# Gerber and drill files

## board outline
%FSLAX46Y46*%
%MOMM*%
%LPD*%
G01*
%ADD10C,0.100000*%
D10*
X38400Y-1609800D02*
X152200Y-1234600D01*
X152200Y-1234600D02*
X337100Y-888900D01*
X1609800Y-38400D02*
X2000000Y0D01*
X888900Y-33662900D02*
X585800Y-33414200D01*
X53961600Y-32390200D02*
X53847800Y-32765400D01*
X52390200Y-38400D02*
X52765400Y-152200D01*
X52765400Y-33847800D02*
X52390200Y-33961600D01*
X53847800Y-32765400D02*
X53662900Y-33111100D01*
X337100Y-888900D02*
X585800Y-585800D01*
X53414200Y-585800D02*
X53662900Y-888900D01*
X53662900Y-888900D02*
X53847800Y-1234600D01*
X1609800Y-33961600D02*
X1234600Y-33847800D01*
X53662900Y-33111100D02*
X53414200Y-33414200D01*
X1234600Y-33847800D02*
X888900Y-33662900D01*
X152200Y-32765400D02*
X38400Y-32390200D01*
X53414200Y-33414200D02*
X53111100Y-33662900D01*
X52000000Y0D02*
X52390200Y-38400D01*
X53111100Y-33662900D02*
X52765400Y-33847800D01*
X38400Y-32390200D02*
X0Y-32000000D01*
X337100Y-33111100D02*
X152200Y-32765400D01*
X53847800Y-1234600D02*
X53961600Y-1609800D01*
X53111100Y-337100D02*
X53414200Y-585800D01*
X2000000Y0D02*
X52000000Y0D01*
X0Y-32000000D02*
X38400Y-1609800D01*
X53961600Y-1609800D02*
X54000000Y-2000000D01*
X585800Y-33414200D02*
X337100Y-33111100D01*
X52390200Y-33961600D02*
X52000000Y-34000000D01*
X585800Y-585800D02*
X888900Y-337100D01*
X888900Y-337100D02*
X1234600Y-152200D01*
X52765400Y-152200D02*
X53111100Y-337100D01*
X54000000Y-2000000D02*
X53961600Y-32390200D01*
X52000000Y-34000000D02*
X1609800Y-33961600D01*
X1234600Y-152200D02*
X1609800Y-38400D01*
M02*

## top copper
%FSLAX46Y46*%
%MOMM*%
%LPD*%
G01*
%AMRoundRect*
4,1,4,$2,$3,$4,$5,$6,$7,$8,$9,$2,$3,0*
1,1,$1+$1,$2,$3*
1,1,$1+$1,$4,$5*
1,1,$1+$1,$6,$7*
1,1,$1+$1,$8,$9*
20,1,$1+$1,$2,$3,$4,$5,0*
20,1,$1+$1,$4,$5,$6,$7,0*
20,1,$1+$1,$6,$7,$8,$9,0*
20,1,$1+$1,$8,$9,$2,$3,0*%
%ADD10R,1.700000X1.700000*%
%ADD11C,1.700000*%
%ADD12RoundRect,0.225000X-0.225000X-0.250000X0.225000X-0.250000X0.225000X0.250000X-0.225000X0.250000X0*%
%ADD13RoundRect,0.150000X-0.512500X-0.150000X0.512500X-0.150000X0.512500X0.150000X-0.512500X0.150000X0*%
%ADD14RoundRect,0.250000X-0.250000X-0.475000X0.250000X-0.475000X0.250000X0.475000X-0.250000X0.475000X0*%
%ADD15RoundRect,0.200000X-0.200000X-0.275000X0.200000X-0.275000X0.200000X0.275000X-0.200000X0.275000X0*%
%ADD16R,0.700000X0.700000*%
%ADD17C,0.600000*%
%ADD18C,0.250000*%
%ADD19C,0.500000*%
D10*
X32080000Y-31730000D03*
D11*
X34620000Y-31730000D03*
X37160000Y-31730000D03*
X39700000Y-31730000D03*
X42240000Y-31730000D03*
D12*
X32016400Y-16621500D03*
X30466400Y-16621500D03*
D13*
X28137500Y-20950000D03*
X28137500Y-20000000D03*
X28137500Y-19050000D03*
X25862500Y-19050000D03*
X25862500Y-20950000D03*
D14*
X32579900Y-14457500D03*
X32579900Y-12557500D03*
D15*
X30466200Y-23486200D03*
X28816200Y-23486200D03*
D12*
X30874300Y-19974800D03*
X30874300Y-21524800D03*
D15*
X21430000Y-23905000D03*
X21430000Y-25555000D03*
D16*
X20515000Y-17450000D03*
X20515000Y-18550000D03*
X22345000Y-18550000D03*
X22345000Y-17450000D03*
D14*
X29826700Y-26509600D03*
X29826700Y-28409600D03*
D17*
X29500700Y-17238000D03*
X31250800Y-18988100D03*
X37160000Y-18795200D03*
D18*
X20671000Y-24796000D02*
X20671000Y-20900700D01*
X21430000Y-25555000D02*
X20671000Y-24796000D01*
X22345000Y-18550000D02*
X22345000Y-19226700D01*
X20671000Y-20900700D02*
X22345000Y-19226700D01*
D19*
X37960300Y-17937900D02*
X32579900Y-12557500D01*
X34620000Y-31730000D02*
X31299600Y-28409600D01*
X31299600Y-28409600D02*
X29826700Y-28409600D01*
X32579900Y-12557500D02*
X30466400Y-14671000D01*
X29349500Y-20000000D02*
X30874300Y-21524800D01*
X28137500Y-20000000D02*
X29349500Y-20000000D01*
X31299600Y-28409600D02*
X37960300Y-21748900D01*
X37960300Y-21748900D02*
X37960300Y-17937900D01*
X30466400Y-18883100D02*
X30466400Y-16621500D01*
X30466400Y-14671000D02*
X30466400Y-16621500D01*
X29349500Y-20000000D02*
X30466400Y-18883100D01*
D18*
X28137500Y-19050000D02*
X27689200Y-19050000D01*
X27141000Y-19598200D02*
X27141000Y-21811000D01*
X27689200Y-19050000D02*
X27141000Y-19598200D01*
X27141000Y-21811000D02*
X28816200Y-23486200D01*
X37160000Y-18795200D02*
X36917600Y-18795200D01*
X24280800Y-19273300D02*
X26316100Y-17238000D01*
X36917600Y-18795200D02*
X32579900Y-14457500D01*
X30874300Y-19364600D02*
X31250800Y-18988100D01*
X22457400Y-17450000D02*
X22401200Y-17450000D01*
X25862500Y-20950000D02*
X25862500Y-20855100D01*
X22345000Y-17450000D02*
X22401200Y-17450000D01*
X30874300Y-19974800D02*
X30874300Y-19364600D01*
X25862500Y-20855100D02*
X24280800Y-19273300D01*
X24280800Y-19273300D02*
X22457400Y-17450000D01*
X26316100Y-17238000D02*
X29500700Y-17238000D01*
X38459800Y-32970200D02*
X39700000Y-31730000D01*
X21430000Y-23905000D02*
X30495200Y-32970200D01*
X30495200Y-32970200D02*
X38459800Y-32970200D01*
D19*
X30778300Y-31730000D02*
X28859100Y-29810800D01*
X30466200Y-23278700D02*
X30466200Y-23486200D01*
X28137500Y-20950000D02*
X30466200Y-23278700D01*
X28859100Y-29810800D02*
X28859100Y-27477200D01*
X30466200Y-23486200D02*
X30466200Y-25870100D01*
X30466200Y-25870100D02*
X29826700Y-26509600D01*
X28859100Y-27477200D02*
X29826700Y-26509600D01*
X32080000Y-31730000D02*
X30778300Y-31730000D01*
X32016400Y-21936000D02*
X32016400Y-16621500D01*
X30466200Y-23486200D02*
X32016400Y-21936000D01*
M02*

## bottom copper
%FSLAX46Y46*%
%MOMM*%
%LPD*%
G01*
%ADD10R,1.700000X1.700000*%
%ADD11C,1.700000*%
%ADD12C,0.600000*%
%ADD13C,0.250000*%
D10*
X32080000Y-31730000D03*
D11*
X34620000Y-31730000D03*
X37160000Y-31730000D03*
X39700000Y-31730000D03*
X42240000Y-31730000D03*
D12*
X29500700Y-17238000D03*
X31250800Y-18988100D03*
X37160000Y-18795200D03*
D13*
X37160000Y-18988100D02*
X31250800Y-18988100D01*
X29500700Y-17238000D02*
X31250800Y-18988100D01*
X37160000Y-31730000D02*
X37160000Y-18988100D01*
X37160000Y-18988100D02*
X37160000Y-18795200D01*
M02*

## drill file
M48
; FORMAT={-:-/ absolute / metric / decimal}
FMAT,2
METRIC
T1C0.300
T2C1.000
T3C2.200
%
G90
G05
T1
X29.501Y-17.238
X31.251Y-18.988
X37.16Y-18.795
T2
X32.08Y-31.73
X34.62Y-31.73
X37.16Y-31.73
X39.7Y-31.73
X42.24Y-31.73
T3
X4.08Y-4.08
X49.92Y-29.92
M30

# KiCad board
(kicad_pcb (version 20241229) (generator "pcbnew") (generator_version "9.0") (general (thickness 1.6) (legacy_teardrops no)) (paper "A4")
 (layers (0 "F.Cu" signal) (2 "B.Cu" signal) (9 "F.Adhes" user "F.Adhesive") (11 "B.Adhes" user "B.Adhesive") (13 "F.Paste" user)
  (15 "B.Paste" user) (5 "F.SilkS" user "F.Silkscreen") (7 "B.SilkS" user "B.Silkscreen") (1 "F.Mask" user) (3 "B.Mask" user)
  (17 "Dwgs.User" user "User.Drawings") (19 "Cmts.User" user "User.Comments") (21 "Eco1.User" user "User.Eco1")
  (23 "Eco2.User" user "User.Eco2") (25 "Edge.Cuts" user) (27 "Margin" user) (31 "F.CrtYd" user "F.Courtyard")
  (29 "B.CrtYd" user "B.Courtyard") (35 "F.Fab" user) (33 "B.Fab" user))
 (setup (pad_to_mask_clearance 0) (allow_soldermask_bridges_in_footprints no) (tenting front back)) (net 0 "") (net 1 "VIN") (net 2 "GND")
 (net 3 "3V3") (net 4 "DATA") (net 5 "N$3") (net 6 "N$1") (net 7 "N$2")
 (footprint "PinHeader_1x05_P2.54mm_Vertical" (layer "F.Cu") (at 32.08 31.73 90)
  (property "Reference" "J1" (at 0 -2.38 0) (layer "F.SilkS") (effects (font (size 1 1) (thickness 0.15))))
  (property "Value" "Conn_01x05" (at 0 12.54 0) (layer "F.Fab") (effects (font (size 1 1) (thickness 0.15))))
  (pad "1" thru_hole rect (at 0 0) (size 1.7 1.7) (drill 1) (layers "*.Cu" "*.Mask") (remove_unused_layers no) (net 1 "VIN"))
  (pad "2" thru_hole circle (at 0 2.54) (size 1.7 1.7) (drill 1) (layers "*.Cu" "*.Mask") (remove_unused_layers no) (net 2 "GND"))
  (pad "3" thru_hole circle (at 0 5.08) (size 1.7 1.7) (drill 1) (layers "*.Cu" "*.Mask") (remove_unused_layers no) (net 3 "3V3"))
  (pad "4" thru_hole circle (at 0 7.62) (size 1.7 1.7) (drill 1) (layers "*.Cu" "*.Mask") (remove_unused_layers no) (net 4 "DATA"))
  (pad "5" thru_hole circle (at 0 10.16) (size 1.7 1.7) (drill 1) (layers "*.Cu" "*.Mask") (remove_unused_layers no) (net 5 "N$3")))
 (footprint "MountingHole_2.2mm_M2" (layer "F.Cu") (at 4.08 4.08)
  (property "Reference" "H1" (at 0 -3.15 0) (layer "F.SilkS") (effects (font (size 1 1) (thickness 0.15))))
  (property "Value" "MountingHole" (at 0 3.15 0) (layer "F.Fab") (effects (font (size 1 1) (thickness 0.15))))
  (pad "" np_thru_hole circle (at 0 0) (size 2.2 2.2) (drill 2.2) (layers "*.Cu" "*.Mask")))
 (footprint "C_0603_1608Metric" (layer "F.Cu") (at 31.2414 16.6215 180)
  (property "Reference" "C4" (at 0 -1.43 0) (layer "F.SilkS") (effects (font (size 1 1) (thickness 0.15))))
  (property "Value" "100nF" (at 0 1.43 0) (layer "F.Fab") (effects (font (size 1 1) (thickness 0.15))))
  (pad "1" smd roundrect (at -0.775 0) (size 0.9 0.95) (layers "F.Cu" "F.Mask" "F.Paste") (roundrect_rratio 0.25) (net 1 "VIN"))
  (pad "2" smd roundrect (at 0.775 0) (size 0.9 0.95) (layers "F.Cu" "F.Mask" "F.Paste") (roundrect_rratio 0.25) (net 2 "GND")))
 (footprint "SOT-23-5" (layer "F.Cu") (at 27 20 180)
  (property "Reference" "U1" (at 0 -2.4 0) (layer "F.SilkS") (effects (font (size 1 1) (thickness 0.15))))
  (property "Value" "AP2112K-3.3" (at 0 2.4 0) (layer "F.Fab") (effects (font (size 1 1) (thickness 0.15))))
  (pad "1" smd roundrect (at -1.1375 -0.95) (size 1.325 0.6) (layers "F.Cu" "F.Mask" "F.Paste") (roundrect_rratio 0.25) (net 1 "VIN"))
  (pad "2" smd roundrect (at -1.1375 0) (size 1.325 0.6) (layers "F.Cu" "F.Mask" "F.Paste") (roundrect_rratio 0.25) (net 2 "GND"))
  (pad "3" smd roundrect (at -1.1375 0.95) (size 1.325 0.6) (layers "F.Cu" "F.Mask" "F.Paste") (roundrect_rratio 0.25) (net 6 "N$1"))
  (pad "4" smd roundrect (at 1.1375 0.95) (size 1.325 0.6) (layers "F.Cu" "F.Mask" "F.Paste") (roundrect_rratio 0.25))
  (pad "5" smd roundrect (at 1.1375 -0.95) (size 1.325 0.6) (layers "F.Cu" "F.Mask" "F.Paste") (roundrect_rratio 0.25) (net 3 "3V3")))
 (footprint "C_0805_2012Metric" (layer "F.Cu") (at 32.5799 13.5075 90)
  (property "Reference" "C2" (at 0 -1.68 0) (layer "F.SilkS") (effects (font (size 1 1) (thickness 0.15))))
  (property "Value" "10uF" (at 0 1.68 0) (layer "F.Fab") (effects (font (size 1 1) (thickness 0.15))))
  (pad "1" smd roundrect (at -0.95 0) (size 1 1.45) (layers "F.Cu" "F.Mask" "F.Paste") (roundrect_rratio 0.25) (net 3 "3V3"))
  (pad "2" smd roundrect (at 0.95 0) (size 1 1.45) (layers "F.Cu" "F.Mask" "F.Paste") (roundrect_rratio 0.25) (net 2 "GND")))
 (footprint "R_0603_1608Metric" (layer "F.Cu") (at 29.6412 23.4862 180)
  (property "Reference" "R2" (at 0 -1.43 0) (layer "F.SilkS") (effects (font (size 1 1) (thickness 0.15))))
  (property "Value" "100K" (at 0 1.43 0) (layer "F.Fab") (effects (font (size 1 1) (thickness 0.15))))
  (pad "1" smd roundrect (at -0.825 0) (size 0.8 0.95) (layers "F.Cu" "F.Mask" "F.Paste") (roundrect_rratio 0.25) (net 1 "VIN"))
  (pad "2" smd roundrect (at 0.825 0) (size 0.8 0.95) (layers "F.Cu" "F.Mask" "F.Paste") (roundrect_rratio 0.25) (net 6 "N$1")))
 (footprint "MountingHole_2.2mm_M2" (layer "F.Cu") (at 49.92 29.92)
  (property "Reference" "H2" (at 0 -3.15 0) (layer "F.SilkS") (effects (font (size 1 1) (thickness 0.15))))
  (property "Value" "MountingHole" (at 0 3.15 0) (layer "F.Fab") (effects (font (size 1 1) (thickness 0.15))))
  (pad "" np_thru_hole circle (at 0 0) (size 2.2 2.2) (drill 2.2) (layers "*.Cu" "*.Mask")))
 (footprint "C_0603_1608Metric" (layer "F.Cu") (at 30.8743 20.7498 -90)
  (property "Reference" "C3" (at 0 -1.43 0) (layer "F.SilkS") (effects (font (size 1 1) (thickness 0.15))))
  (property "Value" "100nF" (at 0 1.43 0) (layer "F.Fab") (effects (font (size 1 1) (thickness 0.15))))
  (pad "1" smd roundrect (at -0.775 0) (size 0.9 0.95) (layers "F.Cu" "F.Mask" "F.Paste") (roundrect_rratio 0.25) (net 3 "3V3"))
  (pad "2" smd roundrect (at 0.775 0) (size 0.9 0.95) (layers "F.Cu" "F.Mask" "F.Paste") (roundrect_rratio 0.25) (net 2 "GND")))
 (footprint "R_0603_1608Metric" (layer "F.Cu") (at 21.43 24.73 -90)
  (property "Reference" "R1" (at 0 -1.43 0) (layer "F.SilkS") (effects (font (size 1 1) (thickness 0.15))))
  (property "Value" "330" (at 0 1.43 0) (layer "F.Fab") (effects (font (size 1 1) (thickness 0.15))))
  (pad "1" smd roundrect (at -0.825 0) (size 0.8 0.95) (layers "F.Cu" "F.Mask" "F.Paste") (roundrect_rratio 0.25) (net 4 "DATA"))
  (pad "2" smd roundrect (at 0.825 0) (size 0.8 0.95) (layers "F.Cu" "F.Mask" "F.Paste") (roundrect_rratio 0.25) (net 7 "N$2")))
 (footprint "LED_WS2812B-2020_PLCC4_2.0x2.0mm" (layer "F.Cu") (at 21.43 18)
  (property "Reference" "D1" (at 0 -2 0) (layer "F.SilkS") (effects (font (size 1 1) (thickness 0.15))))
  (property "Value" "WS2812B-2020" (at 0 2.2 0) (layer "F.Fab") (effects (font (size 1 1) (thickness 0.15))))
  (pad "1" smd rect (at -0.915 -0.55) (size 0.7 0.7) (layers "F.Cu" "F.Mask" "F.Paste") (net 5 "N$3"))
  (pad "2" smd rect (at -0.915 0.55) (size 0.7 0.7) (layers "F.Cu" "F.Mask" "F.Paste") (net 2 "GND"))
  (pad "3" smd rect (at 0.915 0.55) (size 0.7 0.7) (layers "F.Cu" "F.Mask" "F.Paste") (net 7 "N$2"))
  (pad "4" smd rect (at 0.915 -0.55) (size 0.7 0.7) (layers "F.Cu" "F.Mask" "F.Paste") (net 3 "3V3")))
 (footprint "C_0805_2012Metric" (layer "F.Cu") (at 29.8267 27.4596 -90)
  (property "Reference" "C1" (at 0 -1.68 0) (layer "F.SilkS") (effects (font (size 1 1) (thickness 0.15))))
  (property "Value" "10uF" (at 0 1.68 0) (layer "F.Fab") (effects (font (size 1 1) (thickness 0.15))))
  (pad "1" smd roundrect (at -0.95 0) (size 1 1.45) (layers "F.Cu" "F.Mask" "F.Paste") (roundrect_rratio 0.25) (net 1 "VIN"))
  (pad "2" smd roundrect (at 0.95 0) (size 1 1.45) (layers "F.Cu" "F.Mask" "F.Paste") (roundrect_rratio 0.25) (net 2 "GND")))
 (gr_line (start 0.0384 1.6098) (end 0.1522 1.2346) (stroke (width 0.1) (type solid)) (layer "Edge.Cuts"))
 (gr_line (start 0.1522 1.2346) (end 0.3371 0.8889) (stroke (width 0.1) (type solid)) (layer "Edge.Cuts"))
 (gr_line (start 1.6098 0.0384) (end 2 0) (stroke (width 0.1) (type solid)) (layer "Edge.Cuts"))
 (gr_line (start 0.8889 33.6629) (end 0.5858 33.4142) (stroke (width 0.1) (type solid)) (layer "Edge.Cuts"))
 (gr_line (start 53.9616 32.3902) (end 53.8478 32.7654) (stroke (width 0.1) (type solid)) (layer "Edge.Cuts"))
 (gr_line (start 52.3902 0.0384) (end 52.7654 0.1522) (stroke (width 0.1) (type solid)) (layer "Edge.Cuts"))
 (gr_line (start 52.7654 33.8478) (end 52.3902 33.9616) (stroke (width 0.1) (type solid)) (layer "Edge.Cuts"))
 (gr_line (start 53.8478 32.7654) (end 53.6629 33.1111) (stroke (width 0.1) (type solid)) (layer "Edge.Cuts"))
 (gr_line (start 0.3371 0.8889) (end 0.5858 0.5858) (stroke (width 0.1) (type solid)) (layer "Edge.Cuts"))
 (gr_line (start 53.4142 0.5858) (end 53.6629 0.8889) (stroke (width 0.1) (type solid)) (layer "Edge.Cuts"))
 (gr_line (start 53.6629 0.8889) (end 53.8478 1.2346) (stroke (width 0.1) (type solid)) (layer "Edge.Cuts"))
 (gr_line (start 1.6098 33.9616) (end 1.2346 33.8478) (stroke (width 0.1) (type solid)) (layer "Edge.Cuts"))
 (gr_line (start 53.6629 33.1111) (end 53.4142 33.4142) (stroke (width 0.1) (type solid)) (layer "Edge.Cuts"))
 (gr_line (start 1.2346 33.8478) (end 0.8889 33.6629) (stroke (width 0.1) (type solid)) (layer "Edge.Cuts"))
 (gr_line (start 0.1522 32.7654) (end 0.0384 32.3902) (stroke (width 0.1) (type solid)) (layer "Edge.Cuts"))
 (gr_line (start 53.4142 33.4142) (end 53.1111 33.6629) (stroke (width 0.1) (type solid)) (layer "Edge.Cuts"))
 (gr_line (start 52 0) (end 52.3902 0.0384) (stroke (width 0.1) (type solid)) (layer "Edge.Cuts"))
 (gr_line (start 53.1111 33.6629) (end 52.7654 33.8478) (stroke (width 0.1) (type solid)) (layer "Edge.Cuts"))
 (gr_line (start 0.0384 32.3902) (end 0 32) (stroke (width 0.1) (type solid)) (layer "Edge.Cuts"))
 (gr_line (start 0.3371 33.1111) (end 0.1522 32.7654) (stroke (width 0.1) (type solid)) (layer "Edge.Cuts"))
 (gr_line (start 53.8478 1.2346) (end 53.9616 1.6098) (stroke (width 0.1) (type solid)) (layer "Edge.Cuts"))
 (gr_line (start 53.1111 0.3371) (end 53.4142 0.5858) (stroke (width 0.1) (type solid)) (layer "Edge.Cuts"))
 (gr_line (start 2 0) (end 52 0) (stroke (width 0.1) (type solid)) (layer "Edge.Cuts"))
 (gr_line (start 0 32) (end 0.0384 1.6098) (stroke (width 0.1) (type solid)) (layer "Edge.Cuts"))
 (gr_line (start 53.9616 1.6098) (end 54 2) (stroke (width 0.1) (type solid)) (layer "Edge.Cuts"))
 (gr_line (start 0.5858 33.4142) (end 0.3371 33.1111) (stroke (width 0.1) (type solid)) (layer "Edge.Cuts"))
 (gr_line (start 52.3902 33.9616) (end 52 34) (stroke (width 0.1) (type solid)) (layer "Edge.Cuts"))
 (gr_line (start 0.5858 0.5858) (end 0.8889 0.3371) (stroke (width 0.1) (type solid)) (layer "Edge.Cuts"))
 (gr_line (start 0.8889 0.3371) (end 1.2346 0.1522) (stroke (width 0.1) (type solid)) (layer "Edge.Cuts"))
 (gr_line (start 52.7654 0.1522) (end 53.1111 0.3371) (stroke (width 0.1) (type solid)) (layer "Edge.Cuts"))
 (gr_line (start 54 2) (end 53.9616 32.3902) (stroke (width 0.1) (type solid)) (layer "Edge.Cuts"))
 (gr_line (start 52 34) (end 1.6098 33.9616) (stroke (width 0.1) (type solid)) (layer "Edge.Cuts"))
 (gr_line (start 1.2346 0.1522) (end 1.6098 0.0384) (stroke (width 0.1) (type solid)) (layer "Edge.Cuts"))
 (segment (start 20.671 24.796) (end 20.671 20.9007) (width 0.25) (layer "F.Cu") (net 7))
 (segment (start 21.43 25.555) (end 20.671 24.796) (width 0.25) (layer "F.Cu") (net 7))
 (segment (start 22.345 18.55) (end 22.345 19.2267) (width 0.25) (layer "F.Cu") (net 7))
 (segment (start 20.671 20.9007) (end 22.345 19.2267) (width 0.25) (layer "F.Cu") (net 7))
 (segment (start 37.9603 17.9379) (end 32.5799 12.5575) (width 0.5) (layer "F.Cu") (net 2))
 (segment (start 34.62 31.73) (end 31.2996 28.4096) (width 0.5) (layer "F.Cu") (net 2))
 (segment (start 31.2996 28.4096) (end 29.8267 28.4096) (width 0.5) (layer "F.Cu") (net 2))
 (segment (start 32.5799 12.5575) (end 30.4664 14.671) (width 0.5) (layer "F.Cu") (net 2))
 (segment (start 29.3495 20) (end 30.8743 21.5248) (width 0.5) (layer "F.Cu") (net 2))
 (segment (start 28.1375 20) (end 29.3495 20) (width 0.5) (layer "F.Cu") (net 2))
 (segment (start 31.2996 28.4096) (end 37.9603 21.7489) (width 0.5) (layer "F.Cu") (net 2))
 (segment (start 37.9603 21.7489) (end 37.9603 17.9379) (width 0.5) (layer "F.Cu") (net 2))
 (segment (start 30.4664 18.8831) (end 30.4664 16.6215) (width 0.5) (layer "F.Cu") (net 2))
 (segment (start 30.4664 14.671) (end 30.4664 16.6215) (width 0.5) (layer "F.Cu") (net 2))
 (segment (start 29.3495 20) (end 30.4664 18.8831) (width 0.5) (layer "F.Cu") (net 2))
 (segment (start 28.1375 19.05) (end 27.6892 19.05) (width 0.25) (layer "F.Cu") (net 6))
 (segment (start 27.141 19.5982) (end 27.141 21.811) (width 0.25) (layer "F.Cu") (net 6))
 (segment (start 27.6892 19.05) (end 27.141 19.5982) (width 0.25) (layer "F.Cu") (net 6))
 (segment (start 27.141 21.811) (end 28.8162 23.4862) (width 0.25) (layer "F.Cu") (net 6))
 (segment (start 37.16 18.7952) (end 36.9176 18.7952) (width 0.25) (layer "F.Cu") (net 3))
 (segment (start 24.2808 19.2733) (end 26.3161 17.238) (width 0.25) (layer "F.Cu") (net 3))
 (segment (start 36.9176 18.7952) (end 32.5799 14.4575) (width 0.25) (layer "F.Cu") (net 3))
 (segment (start 30.8743 19.3646) (end 31.2508 18.9881) (width 0.25) (layer "F.Cu") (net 3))
 (segment (start 22.4574 17.45) (end 22.4012 17.45) (width 0.25) (layer "F.Cu") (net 3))
 (segment (start 25.8625 20.95) (end 25.8625 20.8551) (width 0.25) (layer "F.Cu") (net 3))
 (segment (start 22.345 17.45) (end 22.4012 17.45) (width 0.25) (layer "F.Cu") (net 3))
 (segment (start 30.8743 19.9748) (end 30.8743 19.3646) (width 0.25) (layer "F.Cu") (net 3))
 (segment (start 25.8625 20.8551) (end 24.2808 19.2733) (width 0.25) (layer "F.Cu") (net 3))
 (segment (start 24.2808 19.2733) (end 22.4574 17.45) (width 0.25) (layer "F.Cu") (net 3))
 (segment (start 26.3161 17.238) (end 29.5007 17.238) (width 0.25) (layer "F.Cu") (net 3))
 (via (at 29.5007 17.238) (size 0.6) (drill 0.3) (layers "F.Cu" "B.Cu") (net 3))
 (via (at 31.2508 18.9881) (size 0.6) (drill 0.3) (layers "F.Cu" "B.Cu") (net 3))
 (via (at 37.16 18.7952) (size 0.6) (drill 0.3) (layers "F.Cu" "B.Cu") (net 3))
 (segment (start 37.16 18.9881) (end 31.2508 18.9881) (width 0.25) (layer "B.Cu") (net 3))
 (segment (start 29.5007 17.238) (end 31.2508 18.9881) (width 0.25) (layer "B.Cu") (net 3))
 (segment (start 37.16 31.73) (end 37.16 18.9881) (width 0.25) (layer "B.Cu") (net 3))
 (segment (start 37.16 18.9881) (end 37.16 18.7952) (width 0.25) (layer "B.Cu") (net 3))
 (segment (start 38.4598 32.9702) (end 39.7 31.73) (width 0.25) (layer "F.Cu") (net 4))
 (segment (start 21.43 23.905) (end 30.4952 32.9702) (width 0.25) (layer "F.Cu") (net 4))
 (segment (start 30.4952 32.9702) (end 38.4598 32.9702) (width 0.25) (layer "F.Cu") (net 4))
 (segment (start 30.7783 31.73) (end 28.8591 29.8108) (width 0.5) (layer "F.Cu") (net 1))
 (segment (start 30.4662 23.2787) (end 30.4662 23.4862) (width 0.5) (layer "F.Cu") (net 1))
 (segment (start 28.1375 20.95) (end 30.4662 23.2787) (width 0.5) (layer "F.Cu") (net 1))
 (segment (start 28.8591 29.8108) (end 28.8591 27.4772) (width 0.5) (layer "F.Cu") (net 1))
 (segment (start 30.4662 23.4862) (end 30.4662 25.8701) (width 0.5) (layer "F.Cu") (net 1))
 (segment (start 30.4662 25.8701) (end 29.8267 26.5096) (width 0.5) (layer "F.Cu") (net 1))
 (segment (start 28.8591 27.4772) (end 29.8267 26.5096) (width 0.5) (layer "F.Cu") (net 1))
 (segment (start 32.08 31.73) (end 30.7783 31.73) (width 0.5) (layer "F.Cu") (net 1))
 (segment (start 32.0164 21.936) (end 32.0164 16.6215) (width 0.5) (layer "F.Cu") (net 1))
 (segment (start 30.4662 23.4862) (end 32.0164 21.936) (width 0.5) (layer "F.Cu") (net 1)))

